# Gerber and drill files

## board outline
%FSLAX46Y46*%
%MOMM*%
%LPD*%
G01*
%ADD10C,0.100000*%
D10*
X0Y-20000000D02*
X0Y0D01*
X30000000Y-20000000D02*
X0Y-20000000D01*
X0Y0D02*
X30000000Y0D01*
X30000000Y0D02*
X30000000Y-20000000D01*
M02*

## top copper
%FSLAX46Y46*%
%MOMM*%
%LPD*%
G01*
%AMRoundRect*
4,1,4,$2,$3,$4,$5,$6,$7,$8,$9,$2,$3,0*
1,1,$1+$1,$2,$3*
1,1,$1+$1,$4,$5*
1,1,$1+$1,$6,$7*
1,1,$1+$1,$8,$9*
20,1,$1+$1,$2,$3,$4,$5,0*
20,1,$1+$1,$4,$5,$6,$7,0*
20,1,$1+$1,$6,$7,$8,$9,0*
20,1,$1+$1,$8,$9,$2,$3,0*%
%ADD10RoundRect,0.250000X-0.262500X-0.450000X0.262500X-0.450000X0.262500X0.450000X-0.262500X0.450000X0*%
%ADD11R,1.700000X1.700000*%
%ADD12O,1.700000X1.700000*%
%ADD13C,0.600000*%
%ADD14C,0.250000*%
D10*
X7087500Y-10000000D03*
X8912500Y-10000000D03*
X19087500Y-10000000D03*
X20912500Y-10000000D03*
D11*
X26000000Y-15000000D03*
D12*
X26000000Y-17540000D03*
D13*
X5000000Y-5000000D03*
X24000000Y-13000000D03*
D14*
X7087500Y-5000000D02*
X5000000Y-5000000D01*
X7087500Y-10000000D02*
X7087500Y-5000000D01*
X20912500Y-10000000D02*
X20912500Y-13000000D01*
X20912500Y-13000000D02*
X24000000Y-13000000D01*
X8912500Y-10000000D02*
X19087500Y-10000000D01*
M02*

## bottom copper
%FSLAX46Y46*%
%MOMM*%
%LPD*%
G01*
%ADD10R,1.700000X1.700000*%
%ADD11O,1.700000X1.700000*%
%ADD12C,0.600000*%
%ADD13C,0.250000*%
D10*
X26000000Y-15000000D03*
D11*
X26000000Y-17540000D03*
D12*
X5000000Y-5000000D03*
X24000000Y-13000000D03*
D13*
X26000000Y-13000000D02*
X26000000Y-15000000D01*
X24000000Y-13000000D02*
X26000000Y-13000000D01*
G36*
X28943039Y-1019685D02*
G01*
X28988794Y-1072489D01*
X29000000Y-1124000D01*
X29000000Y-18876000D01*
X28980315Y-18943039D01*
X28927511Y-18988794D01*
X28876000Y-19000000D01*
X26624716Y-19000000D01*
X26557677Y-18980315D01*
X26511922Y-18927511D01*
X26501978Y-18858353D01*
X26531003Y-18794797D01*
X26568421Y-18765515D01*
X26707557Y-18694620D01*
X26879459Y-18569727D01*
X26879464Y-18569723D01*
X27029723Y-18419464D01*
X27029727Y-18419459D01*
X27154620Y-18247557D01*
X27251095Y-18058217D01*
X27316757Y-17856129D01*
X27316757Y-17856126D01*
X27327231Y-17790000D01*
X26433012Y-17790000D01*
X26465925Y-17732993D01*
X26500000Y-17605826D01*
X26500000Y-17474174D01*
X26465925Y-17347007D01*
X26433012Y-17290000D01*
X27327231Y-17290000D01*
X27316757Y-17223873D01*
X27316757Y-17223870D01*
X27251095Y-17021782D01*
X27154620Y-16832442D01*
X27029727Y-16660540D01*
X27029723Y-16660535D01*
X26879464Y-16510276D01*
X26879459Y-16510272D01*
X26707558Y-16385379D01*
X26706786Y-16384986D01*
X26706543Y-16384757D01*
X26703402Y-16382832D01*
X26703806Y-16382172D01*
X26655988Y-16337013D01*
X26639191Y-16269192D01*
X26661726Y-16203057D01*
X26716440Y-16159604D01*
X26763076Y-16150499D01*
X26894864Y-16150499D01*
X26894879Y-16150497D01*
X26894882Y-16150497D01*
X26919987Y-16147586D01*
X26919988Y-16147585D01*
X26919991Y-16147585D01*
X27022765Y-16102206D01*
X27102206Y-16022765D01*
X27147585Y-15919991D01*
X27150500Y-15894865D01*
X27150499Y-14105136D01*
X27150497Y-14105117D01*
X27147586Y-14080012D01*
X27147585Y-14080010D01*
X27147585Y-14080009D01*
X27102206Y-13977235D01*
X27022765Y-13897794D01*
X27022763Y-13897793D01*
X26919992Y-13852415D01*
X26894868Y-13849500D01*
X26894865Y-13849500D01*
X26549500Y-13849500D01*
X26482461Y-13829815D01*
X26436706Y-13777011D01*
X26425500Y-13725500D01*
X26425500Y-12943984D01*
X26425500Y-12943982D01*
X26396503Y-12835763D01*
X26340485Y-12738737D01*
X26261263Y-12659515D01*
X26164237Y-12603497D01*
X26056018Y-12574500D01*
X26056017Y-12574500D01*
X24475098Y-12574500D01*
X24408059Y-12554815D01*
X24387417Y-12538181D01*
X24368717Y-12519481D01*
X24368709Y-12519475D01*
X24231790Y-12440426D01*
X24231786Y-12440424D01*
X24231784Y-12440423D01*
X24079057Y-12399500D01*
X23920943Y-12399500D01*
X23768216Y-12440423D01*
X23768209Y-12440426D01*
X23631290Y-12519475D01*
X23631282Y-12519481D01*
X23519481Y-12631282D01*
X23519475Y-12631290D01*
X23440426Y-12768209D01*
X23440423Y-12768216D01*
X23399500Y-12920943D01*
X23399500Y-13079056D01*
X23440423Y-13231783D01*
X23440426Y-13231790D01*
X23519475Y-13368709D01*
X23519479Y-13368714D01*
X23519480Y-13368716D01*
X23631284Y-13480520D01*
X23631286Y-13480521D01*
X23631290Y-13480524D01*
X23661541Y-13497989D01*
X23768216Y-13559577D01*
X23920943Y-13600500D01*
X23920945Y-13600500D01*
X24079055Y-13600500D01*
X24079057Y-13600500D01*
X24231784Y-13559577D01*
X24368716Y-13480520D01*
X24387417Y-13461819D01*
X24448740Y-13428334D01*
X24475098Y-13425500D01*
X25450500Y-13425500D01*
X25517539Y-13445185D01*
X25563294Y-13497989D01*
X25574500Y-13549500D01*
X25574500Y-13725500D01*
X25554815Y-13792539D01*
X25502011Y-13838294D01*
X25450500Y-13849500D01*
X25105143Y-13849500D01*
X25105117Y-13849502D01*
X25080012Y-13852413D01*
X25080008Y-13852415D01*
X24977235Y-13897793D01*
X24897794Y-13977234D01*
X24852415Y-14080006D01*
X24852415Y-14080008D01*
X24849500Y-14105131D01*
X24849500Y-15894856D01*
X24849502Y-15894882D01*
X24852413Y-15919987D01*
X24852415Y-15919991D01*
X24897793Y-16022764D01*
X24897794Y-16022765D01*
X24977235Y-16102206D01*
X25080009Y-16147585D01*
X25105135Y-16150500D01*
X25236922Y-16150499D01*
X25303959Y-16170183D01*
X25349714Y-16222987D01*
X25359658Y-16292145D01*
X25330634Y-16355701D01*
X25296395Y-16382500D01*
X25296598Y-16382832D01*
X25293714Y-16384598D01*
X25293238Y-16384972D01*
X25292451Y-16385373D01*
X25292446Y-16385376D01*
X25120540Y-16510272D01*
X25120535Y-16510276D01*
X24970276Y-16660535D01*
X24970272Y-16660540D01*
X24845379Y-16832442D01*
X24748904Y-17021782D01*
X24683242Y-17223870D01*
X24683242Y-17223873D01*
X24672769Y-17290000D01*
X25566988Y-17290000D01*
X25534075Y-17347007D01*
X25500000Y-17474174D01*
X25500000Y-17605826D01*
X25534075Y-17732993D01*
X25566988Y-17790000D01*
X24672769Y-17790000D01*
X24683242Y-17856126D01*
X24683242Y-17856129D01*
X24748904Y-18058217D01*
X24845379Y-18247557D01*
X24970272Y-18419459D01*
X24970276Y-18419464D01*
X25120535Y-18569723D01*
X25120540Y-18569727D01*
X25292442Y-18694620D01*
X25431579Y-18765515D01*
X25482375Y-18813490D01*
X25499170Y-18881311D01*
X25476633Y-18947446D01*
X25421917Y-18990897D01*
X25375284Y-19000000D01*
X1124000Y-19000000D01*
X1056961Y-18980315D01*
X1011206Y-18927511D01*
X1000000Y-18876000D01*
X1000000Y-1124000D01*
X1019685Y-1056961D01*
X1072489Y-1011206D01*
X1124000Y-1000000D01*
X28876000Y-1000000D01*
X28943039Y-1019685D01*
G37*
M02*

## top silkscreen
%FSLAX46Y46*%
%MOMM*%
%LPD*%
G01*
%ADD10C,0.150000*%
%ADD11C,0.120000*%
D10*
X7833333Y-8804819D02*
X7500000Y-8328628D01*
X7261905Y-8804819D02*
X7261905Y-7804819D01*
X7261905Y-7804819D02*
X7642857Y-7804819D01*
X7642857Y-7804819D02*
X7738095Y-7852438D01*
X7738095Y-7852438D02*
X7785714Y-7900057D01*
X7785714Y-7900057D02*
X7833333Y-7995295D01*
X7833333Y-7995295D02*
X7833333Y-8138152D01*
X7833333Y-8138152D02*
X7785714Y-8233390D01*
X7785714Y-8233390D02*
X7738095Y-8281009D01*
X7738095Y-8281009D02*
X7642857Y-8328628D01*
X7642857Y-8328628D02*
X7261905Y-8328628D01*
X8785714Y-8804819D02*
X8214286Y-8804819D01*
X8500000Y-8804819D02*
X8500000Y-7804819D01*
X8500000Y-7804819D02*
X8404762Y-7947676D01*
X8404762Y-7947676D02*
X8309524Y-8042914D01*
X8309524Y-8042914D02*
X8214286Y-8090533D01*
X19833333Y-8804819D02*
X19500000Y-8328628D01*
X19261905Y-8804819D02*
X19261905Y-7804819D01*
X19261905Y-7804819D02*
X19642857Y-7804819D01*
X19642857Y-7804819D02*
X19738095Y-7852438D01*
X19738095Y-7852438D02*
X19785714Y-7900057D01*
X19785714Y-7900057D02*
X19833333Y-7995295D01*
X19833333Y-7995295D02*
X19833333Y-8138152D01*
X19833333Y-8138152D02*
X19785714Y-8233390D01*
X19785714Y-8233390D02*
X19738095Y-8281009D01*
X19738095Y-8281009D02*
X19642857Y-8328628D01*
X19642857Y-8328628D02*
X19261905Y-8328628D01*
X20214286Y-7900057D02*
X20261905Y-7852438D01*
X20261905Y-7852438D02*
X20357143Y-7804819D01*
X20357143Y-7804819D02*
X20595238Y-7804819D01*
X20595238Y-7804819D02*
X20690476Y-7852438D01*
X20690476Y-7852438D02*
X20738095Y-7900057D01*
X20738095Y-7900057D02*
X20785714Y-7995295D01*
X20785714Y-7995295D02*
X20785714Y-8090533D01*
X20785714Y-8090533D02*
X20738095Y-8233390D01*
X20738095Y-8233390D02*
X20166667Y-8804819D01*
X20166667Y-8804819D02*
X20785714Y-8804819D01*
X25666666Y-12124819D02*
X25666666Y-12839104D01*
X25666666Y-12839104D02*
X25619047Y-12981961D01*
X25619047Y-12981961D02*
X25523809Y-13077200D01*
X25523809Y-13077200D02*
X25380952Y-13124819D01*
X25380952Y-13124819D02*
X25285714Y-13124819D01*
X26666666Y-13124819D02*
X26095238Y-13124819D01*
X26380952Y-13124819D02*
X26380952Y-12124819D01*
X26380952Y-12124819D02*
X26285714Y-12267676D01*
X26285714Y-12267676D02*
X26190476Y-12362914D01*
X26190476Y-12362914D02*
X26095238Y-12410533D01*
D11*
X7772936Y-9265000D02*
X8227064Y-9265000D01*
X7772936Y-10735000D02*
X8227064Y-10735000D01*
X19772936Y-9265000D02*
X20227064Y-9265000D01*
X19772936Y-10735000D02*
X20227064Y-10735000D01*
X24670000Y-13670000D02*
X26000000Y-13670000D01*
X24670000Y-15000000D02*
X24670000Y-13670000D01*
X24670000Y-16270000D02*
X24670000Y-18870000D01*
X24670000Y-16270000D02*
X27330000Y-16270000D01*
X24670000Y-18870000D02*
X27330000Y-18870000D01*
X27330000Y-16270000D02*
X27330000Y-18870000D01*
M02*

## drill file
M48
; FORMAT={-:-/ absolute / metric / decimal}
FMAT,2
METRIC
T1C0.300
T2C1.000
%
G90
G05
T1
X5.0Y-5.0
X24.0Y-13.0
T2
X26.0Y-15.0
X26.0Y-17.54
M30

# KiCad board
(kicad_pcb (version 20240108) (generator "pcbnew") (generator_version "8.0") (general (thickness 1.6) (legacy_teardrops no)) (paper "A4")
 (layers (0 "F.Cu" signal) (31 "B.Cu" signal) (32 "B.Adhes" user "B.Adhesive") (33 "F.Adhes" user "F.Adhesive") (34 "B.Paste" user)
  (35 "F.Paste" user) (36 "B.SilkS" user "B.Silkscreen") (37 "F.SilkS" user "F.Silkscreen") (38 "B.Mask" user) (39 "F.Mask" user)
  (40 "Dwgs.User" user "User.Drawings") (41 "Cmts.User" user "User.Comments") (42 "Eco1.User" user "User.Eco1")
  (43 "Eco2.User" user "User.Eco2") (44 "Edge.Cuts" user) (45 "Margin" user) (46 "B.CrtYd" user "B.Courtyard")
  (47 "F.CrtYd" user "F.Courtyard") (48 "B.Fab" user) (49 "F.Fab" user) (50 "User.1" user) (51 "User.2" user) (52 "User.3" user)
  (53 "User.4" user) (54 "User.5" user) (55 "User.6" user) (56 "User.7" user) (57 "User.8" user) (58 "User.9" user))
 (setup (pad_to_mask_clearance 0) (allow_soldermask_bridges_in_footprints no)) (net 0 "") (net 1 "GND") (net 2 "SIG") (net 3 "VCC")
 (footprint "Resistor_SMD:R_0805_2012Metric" (layer "F.Cu") (at 8 10)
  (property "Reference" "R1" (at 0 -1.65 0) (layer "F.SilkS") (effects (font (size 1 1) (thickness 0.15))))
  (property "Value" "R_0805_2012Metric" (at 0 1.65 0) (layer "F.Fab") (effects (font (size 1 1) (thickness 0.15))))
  (fp_line (start -0.227064 -0.735) (end 0.227064 -0.735) (stroke (width 0.12) (type solid)) (layer "F.SilkS"))
  (fp_line (start -0.227064 0.735) (end 0.227064 0.735) (stroke (width 0.12) (type solid)) (layer "F.SilkS"))
  (pad "1" smd roundrect (at -0.9125 0) (size 1.025 1.4) (layers "F.Cu" "F.Paste" "F.Mask") (roundrect_rratio 0.243902) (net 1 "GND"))
  (pad "2" smd roundrect (at 0.9125 0) (size 1.025 1.4) (layers "F.Cu" "F.Paste" "F.Mask") (roundrect_rratio 0.243902) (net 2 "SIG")))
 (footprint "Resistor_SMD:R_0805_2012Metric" (layer "F.Cu") (at 20 10)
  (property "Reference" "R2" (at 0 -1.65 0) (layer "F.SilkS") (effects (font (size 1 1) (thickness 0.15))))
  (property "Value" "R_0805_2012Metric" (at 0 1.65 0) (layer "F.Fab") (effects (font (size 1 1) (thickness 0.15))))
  (fp_line (start -0.227064 -0.735) (end 0.227064 -0.735) (stroke (width 0.12) (type solid)) (layer "F.SilkS"))
  (fp_line (start -0.227064 0.735) (end 0.227064 0.735) (stroke (width 0.12) (type solid)) (layer "F.SilkS"))
  (pad "1" smd roundrect (at -0.9125 0) (size 1.025 1.4) (layers "F.Cu" "F.Paste" "F.Mask") (roundrect_rratio 0.243902) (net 2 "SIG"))
  (pad "2" smd roundrect (at 0.9125 0) (size 1.025 1.4) (layers "F.Cu" "F.Paste" "F.Mask") (roundrect_rratio 0.243902) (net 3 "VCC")))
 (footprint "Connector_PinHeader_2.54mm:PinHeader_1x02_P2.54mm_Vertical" (layer "F.Cu") (at 26 15)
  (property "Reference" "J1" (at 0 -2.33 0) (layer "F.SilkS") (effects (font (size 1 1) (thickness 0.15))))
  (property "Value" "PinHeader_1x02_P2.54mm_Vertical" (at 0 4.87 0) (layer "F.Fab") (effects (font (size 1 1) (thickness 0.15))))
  (fp_line (start -1.33 -1.33) (end 0 -1.33) (stroke (width 0.12) (type solid)) (layer "F.SilkS"))
  (fp_line (start -1.33 0) (end -1.33 -1.33) (stroke (width 0.12) (type solid)) (layer "F.SilkS"))
  (fp_line (start -1.33 1.27) (end -1.33 3.87) (stroke (width 0.12) (type solid)) (layer "F.SilkS"))
  (fp_line (start -1.33 1.27) (end 1.33 1.27) (stroke (width 0.12) (type solid)) (layer "F.SilkS"))
  (fp_line (start -1.33 3.87) (end 1.33 3.87) (stroke (width 0.12) (type solid)) (layer "F.SilkS"))
  (fp_line (start 1.33 1.27) (end 1.33 3.87) (stroke (width 0.12) (type solid)) (layer "F.SilkS"))
  (pad "1" thru_hole rect (at 0 0) (size 1.7 1.7) (drill 1) (layers "*.Cu" "*.Mask") (remove_unused_layers no) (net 3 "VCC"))
  (pad "2" thru_hole oval (at 0 2.54) (size 1.7 1.7) (drill 1) (layers "*.Cu" "*.Mask") (remove_unused_layers no) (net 1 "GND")))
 (gr_line (start 0 20) (end 0 0) (stroke (width 0.1) (type default)) (layer "Edge.Cuts"))
 (gr_line (start 30 20) (end 0 20) (stroke (width 0.1) (type default)) (layer "Edge.Cuts"))
 (gr_line (start 0 0) (end 30 0) (stroke (width 0.1) (type default)) (layer "Edge.Cuts"))
 (gr_line (start 30 0) (end 30 20) (stroke (width 0.1) (type default)) (layer "Edge.Cuts"))
 (segment (start 7.0875 5) (end 5 5) (width 0.25) (layer "F.Cu") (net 1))
 (segment (start 7.0875 10) (end 7.0875 5) (width 0.25) (layer "F.Cu") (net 1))
 (via (at 5 5) (size 0.6) (drill 0.3) (layers "F.Cu" "B.Cu") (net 1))
 (segment (start 20.9125 10) (end 20.9125 13) (width 0.25) (layer "F.Cu") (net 3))
 (segment (start 20.9125 13) (end 24 13) (width 0.25) (layer "F.Cu") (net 3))
 (via (at 24 13) (size 0.6) (drill 0.3) (layers "F.Cu" "B.Cu") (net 3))
 (segment (start 26 13) (end 26 15) (width 0.25) (layer "B.Cu") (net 3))
 (segment (start 24 13) (end 26 13) (width 0.25) (layer "B.Cu") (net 3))
 (segment (start 8.9125 10) (end 19.0875 10) (width 0.25) (layer "F.Cu") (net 2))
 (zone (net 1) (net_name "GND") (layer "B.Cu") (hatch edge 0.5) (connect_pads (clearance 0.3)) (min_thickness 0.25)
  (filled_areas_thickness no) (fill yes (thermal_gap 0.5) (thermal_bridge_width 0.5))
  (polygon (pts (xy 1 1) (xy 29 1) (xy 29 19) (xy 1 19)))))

